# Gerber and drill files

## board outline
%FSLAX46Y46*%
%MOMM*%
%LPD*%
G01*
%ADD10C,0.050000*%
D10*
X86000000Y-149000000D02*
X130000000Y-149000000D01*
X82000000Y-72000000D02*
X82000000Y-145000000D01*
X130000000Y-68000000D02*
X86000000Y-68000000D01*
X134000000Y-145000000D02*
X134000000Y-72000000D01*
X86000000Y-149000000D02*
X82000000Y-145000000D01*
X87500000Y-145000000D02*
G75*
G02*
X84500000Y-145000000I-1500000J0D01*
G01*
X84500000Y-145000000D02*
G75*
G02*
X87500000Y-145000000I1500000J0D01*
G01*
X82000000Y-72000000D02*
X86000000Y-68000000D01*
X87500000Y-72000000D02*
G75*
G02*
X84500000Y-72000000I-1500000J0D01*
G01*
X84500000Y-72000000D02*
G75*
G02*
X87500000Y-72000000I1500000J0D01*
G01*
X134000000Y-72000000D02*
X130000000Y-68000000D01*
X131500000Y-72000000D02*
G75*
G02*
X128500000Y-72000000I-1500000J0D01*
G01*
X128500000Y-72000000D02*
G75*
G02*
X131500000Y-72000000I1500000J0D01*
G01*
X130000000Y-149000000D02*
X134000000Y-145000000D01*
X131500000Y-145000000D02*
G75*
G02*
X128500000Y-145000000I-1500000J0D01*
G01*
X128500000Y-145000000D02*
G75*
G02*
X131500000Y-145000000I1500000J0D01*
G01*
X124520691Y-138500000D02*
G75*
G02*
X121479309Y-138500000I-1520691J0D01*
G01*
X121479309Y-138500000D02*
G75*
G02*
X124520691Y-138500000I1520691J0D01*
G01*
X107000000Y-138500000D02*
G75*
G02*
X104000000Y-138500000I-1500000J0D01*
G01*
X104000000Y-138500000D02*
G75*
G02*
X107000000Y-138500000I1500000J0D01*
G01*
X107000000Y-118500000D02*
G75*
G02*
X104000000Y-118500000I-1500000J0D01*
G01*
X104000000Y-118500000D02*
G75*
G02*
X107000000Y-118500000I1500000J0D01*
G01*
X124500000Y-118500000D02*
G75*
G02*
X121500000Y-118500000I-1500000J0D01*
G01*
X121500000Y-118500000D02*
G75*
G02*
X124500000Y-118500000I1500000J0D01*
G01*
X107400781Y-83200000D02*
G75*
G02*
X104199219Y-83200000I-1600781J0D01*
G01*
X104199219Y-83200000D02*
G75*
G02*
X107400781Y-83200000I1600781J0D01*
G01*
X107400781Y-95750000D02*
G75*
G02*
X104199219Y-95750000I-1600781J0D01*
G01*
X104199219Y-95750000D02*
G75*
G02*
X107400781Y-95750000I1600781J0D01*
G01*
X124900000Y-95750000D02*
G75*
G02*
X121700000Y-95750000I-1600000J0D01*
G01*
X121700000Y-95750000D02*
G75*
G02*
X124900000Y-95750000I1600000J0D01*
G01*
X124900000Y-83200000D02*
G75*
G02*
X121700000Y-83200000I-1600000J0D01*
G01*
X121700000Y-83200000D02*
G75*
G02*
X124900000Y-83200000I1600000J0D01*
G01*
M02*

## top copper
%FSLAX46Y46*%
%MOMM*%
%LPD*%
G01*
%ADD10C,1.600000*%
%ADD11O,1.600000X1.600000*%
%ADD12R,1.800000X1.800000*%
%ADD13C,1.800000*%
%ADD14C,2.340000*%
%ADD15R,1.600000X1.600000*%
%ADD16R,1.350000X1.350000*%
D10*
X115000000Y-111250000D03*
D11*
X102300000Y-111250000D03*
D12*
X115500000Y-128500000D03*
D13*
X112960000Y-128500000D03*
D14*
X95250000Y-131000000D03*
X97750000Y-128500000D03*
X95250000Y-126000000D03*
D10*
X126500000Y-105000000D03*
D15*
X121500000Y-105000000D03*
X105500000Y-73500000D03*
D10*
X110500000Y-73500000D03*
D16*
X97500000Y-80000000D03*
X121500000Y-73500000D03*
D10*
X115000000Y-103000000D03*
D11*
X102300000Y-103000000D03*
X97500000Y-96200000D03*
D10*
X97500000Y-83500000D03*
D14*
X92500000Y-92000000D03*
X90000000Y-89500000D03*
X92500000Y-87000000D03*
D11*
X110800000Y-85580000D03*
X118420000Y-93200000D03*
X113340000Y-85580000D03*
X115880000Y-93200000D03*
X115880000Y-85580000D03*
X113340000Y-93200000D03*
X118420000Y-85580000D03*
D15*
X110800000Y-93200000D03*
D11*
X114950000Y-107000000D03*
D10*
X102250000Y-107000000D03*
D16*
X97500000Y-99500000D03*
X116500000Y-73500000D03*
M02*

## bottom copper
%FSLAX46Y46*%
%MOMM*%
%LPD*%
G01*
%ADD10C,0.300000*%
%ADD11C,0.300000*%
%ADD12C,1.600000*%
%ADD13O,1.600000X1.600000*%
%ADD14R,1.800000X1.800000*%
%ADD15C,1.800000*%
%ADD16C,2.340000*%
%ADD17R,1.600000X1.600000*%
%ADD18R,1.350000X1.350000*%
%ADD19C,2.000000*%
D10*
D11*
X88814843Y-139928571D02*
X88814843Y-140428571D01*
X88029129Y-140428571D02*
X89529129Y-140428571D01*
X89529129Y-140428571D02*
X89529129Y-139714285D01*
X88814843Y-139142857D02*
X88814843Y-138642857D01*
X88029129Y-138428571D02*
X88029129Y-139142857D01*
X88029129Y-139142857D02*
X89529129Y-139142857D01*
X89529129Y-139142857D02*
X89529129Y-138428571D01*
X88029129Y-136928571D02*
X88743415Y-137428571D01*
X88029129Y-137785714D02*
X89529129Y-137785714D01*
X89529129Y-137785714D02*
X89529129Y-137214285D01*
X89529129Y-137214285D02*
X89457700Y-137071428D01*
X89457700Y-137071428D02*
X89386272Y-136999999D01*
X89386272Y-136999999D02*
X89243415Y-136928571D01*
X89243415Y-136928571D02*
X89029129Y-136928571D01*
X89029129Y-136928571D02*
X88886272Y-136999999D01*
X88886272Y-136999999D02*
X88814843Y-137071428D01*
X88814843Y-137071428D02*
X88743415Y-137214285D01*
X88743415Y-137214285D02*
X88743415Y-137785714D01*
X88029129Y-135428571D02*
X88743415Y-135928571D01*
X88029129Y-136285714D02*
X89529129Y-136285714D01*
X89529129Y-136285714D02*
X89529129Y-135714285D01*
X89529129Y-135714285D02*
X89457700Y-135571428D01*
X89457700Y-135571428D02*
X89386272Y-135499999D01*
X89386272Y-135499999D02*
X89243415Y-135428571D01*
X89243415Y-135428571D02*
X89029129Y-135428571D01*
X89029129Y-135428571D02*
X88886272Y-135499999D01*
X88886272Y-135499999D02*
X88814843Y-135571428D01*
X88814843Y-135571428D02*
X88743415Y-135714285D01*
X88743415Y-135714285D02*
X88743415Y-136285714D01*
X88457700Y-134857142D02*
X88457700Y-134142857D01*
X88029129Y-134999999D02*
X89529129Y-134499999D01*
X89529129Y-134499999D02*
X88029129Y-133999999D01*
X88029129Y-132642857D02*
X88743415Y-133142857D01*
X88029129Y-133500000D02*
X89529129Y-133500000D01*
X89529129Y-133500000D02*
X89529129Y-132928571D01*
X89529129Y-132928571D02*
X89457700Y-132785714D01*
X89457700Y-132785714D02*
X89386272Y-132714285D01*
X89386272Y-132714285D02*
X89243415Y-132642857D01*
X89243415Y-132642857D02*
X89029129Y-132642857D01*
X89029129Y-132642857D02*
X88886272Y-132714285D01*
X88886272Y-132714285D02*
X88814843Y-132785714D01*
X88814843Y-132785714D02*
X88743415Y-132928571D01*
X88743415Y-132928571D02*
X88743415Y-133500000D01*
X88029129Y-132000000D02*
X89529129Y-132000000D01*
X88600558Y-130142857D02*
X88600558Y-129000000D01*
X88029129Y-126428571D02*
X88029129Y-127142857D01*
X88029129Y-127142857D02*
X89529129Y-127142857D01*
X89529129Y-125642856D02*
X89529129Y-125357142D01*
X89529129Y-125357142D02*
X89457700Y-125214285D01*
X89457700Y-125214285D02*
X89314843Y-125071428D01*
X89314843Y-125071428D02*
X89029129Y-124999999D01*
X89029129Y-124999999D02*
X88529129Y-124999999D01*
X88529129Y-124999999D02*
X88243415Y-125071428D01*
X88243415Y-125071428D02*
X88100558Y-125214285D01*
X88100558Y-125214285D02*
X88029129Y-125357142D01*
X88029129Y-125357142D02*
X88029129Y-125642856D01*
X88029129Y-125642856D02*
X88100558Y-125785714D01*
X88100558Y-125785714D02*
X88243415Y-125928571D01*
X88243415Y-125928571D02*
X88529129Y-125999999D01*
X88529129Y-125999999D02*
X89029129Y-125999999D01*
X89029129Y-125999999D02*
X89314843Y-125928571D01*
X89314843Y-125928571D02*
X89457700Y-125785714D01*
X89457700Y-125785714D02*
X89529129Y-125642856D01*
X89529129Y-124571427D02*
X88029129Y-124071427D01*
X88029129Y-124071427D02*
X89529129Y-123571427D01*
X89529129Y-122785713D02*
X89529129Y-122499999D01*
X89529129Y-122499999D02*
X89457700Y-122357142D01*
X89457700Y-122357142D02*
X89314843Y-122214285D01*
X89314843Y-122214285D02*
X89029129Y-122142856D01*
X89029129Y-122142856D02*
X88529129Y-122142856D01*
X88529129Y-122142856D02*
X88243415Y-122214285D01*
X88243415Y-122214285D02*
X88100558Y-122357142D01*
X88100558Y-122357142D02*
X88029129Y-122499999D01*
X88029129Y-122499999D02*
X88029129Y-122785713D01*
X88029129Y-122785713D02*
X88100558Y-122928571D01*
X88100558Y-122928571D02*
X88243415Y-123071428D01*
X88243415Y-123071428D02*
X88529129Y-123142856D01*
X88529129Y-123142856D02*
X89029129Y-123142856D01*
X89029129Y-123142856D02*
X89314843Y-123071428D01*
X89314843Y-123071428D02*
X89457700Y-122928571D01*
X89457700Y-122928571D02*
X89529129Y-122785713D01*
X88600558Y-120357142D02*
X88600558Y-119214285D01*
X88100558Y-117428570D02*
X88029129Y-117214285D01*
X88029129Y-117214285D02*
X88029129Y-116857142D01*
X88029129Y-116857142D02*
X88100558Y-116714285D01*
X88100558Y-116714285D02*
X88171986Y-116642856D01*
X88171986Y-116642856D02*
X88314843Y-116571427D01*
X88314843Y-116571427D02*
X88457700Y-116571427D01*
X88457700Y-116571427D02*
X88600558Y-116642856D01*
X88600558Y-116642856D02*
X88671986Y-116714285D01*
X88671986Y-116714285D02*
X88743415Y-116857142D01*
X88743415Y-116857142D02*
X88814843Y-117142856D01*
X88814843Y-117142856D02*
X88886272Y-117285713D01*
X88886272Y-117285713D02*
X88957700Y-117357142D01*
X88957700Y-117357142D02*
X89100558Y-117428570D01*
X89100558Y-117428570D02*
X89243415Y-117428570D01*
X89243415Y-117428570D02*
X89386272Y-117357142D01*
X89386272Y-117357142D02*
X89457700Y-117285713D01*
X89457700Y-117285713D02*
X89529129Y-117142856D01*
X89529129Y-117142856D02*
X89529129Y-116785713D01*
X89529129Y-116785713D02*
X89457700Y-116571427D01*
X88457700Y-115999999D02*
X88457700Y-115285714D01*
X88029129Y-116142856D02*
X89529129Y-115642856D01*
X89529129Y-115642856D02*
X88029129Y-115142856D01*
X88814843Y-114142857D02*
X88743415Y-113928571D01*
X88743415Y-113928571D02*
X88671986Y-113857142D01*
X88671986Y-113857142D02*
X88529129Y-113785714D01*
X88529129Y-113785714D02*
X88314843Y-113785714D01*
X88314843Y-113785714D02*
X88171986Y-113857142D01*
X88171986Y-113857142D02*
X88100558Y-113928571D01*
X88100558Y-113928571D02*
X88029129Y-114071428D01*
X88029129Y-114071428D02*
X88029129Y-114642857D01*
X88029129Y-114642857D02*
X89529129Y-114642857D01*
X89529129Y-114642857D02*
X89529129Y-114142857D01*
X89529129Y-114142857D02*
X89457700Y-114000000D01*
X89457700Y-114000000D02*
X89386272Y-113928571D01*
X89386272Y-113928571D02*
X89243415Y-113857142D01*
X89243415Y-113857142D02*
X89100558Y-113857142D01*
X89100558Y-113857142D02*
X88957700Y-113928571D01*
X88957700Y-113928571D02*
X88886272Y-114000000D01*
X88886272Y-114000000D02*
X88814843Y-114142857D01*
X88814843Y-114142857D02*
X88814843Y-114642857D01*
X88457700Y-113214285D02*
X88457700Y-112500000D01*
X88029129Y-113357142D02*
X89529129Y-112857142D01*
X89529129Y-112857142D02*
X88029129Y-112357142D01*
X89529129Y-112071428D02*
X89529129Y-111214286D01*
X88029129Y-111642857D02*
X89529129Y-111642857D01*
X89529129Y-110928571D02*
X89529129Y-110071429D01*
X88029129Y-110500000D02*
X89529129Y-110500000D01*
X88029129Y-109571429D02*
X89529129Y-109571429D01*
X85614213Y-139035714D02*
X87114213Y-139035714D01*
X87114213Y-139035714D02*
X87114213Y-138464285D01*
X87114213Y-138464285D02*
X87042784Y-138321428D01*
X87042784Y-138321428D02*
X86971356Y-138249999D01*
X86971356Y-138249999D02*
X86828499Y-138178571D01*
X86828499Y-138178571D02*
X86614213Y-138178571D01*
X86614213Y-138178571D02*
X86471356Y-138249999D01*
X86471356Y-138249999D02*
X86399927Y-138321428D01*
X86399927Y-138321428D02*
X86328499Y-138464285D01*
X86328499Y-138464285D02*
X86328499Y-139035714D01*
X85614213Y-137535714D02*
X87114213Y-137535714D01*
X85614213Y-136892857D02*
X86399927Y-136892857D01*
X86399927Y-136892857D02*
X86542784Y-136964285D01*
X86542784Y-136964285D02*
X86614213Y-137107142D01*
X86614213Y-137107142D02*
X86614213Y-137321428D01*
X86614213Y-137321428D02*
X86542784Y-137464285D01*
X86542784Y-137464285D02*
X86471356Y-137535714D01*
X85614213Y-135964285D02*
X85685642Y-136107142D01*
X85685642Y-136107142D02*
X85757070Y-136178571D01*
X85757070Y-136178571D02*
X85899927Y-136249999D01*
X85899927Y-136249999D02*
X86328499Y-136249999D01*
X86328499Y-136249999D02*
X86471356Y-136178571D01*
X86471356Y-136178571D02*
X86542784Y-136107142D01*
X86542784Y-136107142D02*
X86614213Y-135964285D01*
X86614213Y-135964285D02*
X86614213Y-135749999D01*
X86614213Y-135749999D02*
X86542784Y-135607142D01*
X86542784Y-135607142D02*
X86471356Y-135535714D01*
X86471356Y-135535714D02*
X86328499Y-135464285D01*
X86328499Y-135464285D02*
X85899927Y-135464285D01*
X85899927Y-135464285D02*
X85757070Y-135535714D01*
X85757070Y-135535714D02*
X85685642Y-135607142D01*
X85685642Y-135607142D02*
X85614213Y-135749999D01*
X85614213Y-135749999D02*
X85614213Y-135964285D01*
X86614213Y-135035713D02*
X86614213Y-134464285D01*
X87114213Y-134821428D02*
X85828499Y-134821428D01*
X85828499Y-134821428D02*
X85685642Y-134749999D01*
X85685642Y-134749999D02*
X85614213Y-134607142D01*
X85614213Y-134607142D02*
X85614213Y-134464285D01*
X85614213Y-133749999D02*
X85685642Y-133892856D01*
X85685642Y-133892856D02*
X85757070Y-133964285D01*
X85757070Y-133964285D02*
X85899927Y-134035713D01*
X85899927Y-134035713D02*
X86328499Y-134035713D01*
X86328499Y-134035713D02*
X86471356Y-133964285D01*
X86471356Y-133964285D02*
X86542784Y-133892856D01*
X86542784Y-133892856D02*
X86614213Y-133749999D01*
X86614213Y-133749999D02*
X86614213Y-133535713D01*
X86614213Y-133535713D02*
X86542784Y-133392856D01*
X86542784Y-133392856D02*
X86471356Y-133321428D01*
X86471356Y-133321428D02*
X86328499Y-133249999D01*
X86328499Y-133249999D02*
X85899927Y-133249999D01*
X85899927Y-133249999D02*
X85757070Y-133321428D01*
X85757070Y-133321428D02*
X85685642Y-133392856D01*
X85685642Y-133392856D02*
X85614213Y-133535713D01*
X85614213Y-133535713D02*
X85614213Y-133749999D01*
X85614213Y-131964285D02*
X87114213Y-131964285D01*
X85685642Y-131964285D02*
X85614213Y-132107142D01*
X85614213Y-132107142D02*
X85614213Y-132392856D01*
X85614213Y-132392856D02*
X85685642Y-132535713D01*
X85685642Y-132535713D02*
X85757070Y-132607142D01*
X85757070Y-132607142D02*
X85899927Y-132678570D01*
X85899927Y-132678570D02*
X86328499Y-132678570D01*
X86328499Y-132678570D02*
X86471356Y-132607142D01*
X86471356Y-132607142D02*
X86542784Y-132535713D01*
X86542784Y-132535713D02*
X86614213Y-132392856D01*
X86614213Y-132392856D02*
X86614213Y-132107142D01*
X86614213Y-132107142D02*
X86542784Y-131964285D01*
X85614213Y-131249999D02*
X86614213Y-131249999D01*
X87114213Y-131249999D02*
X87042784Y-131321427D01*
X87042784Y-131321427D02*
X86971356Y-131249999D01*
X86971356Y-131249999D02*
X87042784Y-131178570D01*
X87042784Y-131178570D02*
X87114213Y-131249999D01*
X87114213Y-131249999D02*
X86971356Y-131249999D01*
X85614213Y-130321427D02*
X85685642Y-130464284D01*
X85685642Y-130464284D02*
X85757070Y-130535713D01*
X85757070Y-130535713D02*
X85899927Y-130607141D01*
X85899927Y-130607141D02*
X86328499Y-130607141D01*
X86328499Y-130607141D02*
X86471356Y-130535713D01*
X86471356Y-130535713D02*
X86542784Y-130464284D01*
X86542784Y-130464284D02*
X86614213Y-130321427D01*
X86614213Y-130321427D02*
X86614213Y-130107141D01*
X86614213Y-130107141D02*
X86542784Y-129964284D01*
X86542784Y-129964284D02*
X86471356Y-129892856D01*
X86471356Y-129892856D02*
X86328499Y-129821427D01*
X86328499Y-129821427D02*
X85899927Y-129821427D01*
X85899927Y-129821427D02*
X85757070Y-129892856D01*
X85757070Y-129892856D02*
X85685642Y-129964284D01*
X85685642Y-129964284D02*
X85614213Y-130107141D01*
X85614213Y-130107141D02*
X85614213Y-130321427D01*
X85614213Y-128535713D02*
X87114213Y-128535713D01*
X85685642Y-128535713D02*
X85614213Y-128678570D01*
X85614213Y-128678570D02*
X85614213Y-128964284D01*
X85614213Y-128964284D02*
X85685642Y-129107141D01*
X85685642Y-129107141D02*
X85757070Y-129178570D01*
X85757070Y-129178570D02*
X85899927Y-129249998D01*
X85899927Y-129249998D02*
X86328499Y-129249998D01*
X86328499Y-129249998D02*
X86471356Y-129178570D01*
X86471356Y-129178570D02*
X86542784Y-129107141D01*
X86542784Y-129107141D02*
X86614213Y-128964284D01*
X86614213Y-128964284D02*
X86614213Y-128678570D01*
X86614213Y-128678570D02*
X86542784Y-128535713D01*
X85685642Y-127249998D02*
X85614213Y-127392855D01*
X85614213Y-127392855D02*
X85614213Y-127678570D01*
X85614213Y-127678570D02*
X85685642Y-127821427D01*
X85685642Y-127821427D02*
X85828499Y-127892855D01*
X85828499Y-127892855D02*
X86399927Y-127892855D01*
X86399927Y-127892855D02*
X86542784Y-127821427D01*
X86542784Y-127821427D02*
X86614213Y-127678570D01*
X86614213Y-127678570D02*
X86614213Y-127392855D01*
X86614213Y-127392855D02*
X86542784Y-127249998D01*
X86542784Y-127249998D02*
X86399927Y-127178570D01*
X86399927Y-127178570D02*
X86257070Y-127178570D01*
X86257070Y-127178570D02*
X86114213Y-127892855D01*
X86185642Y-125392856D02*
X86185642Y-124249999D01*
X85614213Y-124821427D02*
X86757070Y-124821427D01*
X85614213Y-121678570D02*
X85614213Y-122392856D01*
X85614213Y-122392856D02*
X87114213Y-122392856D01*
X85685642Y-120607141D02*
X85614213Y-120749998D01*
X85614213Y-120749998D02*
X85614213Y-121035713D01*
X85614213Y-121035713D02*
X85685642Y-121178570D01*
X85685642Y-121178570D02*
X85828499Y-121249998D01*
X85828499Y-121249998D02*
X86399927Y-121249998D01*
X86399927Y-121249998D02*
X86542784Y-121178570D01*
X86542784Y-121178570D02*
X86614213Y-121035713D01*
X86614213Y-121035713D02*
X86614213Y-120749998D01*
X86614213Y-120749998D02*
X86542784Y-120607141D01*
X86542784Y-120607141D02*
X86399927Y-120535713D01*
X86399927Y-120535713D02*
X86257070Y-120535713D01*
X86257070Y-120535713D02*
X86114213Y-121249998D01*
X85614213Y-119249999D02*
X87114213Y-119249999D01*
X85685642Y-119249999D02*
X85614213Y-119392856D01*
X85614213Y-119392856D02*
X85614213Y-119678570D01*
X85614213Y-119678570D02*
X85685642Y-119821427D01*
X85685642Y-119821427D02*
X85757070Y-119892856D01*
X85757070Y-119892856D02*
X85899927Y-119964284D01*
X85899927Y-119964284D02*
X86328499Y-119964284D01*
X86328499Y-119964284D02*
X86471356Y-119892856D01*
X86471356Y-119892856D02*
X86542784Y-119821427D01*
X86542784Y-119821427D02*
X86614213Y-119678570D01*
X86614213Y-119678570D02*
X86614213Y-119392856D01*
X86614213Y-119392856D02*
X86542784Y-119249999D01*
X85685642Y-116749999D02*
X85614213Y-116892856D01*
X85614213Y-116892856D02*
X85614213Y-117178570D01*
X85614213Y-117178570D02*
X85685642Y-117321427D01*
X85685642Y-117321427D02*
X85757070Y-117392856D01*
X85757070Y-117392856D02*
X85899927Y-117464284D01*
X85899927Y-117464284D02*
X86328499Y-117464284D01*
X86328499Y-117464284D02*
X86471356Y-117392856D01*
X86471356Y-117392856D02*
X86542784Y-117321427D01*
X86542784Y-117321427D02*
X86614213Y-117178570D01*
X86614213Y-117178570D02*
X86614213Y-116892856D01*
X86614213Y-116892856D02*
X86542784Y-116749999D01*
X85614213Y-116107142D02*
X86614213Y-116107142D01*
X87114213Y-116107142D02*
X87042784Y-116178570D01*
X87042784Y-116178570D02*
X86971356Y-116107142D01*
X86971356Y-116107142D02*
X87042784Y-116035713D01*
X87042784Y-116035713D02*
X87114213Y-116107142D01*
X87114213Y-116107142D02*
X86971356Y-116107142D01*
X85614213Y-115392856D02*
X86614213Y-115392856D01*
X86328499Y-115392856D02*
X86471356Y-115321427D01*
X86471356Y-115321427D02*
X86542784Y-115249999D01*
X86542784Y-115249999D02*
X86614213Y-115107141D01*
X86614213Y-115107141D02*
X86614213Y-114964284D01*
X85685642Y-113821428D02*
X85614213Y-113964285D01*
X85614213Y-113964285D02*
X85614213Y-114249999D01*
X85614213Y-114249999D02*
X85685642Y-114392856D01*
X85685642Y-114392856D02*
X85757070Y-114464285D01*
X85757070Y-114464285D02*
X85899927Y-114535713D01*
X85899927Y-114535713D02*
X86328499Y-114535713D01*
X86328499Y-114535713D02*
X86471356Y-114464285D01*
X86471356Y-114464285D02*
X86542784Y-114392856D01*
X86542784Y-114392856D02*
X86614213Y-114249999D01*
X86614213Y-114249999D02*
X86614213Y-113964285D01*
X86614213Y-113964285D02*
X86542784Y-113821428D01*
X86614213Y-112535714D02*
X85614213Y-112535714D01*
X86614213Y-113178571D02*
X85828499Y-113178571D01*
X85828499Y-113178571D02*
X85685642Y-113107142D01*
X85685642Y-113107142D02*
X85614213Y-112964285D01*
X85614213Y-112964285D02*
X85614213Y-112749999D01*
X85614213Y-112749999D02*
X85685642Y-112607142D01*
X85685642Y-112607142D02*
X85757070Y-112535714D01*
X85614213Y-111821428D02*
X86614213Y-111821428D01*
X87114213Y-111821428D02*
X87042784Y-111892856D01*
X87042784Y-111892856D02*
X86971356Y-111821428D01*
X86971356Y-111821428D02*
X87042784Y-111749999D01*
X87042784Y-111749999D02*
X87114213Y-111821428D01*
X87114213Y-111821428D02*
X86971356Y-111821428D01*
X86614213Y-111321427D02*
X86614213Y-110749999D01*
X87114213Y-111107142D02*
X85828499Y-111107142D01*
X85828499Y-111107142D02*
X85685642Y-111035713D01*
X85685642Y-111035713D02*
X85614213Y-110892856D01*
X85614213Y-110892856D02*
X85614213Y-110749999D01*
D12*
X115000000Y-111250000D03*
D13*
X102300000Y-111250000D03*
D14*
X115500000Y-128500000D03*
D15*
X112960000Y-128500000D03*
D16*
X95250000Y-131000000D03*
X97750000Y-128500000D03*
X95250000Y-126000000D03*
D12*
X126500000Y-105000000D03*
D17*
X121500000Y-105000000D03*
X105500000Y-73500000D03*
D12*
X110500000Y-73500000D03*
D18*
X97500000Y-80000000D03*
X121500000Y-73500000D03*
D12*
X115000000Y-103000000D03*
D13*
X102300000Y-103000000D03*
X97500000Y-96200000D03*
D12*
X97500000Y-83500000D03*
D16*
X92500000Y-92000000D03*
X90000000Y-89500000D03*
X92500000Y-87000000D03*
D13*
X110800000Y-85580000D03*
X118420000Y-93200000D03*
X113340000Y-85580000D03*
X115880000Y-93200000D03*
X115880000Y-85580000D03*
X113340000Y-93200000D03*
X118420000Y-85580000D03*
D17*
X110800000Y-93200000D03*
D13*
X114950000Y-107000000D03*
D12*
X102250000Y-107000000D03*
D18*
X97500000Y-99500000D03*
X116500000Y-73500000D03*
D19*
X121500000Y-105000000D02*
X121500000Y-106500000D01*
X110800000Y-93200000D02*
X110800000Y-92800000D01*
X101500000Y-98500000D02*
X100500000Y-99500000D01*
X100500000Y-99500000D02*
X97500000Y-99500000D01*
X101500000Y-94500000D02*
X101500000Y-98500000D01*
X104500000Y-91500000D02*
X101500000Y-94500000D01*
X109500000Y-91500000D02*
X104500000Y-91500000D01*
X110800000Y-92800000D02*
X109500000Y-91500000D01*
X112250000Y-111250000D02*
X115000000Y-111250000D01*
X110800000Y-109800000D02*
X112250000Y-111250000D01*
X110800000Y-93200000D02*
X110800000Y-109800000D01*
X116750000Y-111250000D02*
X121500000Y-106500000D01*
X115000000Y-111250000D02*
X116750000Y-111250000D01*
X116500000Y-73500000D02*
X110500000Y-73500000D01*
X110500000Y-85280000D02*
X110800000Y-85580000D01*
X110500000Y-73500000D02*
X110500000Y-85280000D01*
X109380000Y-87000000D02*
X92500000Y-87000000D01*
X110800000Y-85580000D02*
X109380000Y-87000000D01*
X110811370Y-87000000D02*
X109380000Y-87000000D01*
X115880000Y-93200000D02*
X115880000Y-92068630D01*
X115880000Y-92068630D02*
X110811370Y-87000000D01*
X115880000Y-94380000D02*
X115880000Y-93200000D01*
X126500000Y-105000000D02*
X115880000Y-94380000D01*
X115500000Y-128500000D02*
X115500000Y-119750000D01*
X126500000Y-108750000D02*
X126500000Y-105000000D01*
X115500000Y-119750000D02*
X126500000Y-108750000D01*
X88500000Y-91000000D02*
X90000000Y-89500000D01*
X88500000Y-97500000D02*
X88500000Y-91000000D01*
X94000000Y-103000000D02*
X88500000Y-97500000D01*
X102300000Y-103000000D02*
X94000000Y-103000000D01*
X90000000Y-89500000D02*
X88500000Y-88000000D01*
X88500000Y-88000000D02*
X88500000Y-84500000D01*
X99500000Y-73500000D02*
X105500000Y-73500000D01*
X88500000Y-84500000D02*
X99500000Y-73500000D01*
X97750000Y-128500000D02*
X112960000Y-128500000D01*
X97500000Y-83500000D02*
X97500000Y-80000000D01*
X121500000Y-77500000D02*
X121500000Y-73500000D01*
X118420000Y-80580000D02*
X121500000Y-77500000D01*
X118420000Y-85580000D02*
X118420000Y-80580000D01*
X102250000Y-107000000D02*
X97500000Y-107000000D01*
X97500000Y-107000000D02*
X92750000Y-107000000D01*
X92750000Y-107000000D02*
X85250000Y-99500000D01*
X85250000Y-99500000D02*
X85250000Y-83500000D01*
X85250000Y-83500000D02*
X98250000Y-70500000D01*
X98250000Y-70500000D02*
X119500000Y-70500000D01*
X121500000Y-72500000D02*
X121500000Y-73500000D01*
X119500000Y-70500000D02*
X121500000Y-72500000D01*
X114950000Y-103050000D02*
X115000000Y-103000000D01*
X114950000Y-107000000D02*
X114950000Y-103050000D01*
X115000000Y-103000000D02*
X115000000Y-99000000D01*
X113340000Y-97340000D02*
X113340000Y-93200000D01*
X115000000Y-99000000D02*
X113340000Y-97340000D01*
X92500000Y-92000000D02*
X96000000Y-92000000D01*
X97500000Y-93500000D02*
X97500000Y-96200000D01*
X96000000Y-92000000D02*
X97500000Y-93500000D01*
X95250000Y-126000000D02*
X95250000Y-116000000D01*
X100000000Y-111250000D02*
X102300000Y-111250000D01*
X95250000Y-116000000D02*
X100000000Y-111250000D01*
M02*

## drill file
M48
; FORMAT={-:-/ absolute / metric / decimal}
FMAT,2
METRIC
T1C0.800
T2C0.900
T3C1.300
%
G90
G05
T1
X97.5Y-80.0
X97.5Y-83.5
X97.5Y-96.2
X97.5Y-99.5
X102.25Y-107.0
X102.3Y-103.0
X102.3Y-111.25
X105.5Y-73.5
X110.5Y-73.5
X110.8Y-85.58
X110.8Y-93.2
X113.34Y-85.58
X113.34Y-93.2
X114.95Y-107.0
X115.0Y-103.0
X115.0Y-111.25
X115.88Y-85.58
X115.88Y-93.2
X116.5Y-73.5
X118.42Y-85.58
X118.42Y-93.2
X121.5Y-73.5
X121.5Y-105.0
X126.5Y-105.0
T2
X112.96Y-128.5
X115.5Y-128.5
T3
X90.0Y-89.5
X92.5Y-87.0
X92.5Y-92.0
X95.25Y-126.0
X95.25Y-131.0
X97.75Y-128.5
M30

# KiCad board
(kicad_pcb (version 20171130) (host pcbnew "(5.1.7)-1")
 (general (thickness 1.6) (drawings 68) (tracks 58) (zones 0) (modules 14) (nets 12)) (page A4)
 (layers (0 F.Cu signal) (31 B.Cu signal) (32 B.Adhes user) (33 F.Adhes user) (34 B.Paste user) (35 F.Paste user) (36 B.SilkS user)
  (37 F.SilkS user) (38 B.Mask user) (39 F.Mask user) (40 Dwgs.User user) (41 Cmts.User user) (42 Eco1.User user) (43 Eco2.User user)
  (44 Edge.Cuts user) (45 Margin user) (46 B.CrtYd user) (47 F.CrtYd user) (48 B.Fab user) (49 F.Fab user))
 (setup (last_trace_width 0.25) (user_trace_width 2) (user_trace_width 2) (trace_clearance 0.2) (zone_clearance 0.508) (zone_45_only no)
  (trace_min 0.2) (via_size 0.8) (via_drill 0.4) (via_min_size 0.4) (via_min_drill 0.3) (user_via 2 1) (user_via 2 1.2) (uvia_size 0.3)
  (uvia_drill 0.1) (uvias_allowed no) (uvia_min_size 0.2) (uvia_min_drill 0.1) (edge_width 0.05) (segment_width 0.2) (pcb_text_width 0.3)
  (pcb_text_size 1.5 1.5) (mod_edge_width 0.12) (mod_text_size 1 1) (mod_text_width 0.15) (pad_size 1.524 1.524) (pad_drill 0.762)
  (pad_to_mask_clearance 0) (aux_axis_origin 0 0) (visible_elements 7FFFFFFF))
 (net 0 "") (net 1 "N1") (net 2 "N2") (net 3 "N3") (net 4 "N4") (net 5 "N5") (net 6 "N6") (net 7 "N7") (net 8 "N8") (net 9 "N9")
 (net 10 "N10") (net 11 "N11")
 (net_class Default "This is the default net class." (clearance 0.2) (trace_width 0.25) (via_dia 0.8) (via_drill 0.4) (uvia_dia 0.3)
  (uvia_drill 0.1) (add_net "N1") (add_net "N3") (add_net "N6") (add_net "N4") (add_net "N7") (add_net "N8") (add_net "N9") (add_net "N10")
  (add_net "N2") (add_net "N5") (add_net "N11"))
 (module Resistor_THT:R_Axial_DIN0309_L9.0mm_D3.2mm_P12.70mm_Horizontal (layer F.Cu) (at 115 111.25 180)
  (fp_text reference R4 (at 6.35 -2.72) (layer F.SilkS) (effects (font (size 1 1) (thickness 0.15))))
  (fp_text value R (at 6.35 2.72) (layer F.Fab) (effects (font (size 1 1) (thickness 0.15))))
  (pad 1 thru_hole circle (at 0 0 180) (size 1.6 1.6) (drill 0.8) (layers *.Cu *.Mask) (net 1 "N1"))
  (pad 2 thru_hole oval (at 12.7 0 180) (size 1.6 1.6) (drill 0.8) (layers *.Cu *.Mask) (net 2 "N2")))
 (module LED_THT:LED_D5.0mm (layer F.Cu) (at 115.5 128.5 180)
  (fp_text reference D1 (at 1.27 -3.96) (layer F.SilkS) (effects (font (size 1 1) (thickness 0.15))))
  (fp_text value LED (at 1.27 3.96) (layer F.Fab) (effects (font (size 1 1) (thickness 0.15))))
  (pad 1 thru_hole rect (at 0 0 180) (size 1.8 1.8) (drill 0.9) (layers *.Cu *.Mask) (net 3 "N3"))
  (pad 2 thru_hole circle (at 2.54 0 180) (size 1.8 1.8) (drill 0.9) (layers *.Cu *.Mask) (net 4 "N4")))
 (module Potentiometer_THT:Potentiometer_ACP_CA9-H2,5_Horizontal (layer F.Cu) (at 95.25 126)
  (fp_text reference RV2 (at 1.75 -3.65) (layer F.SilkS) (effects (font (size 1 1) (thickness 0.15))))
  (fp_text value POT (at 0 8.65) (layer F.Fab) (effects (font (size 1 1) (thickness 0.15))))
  (pad 3 thru_hole circle (at 0 5) (size 2.34 2.34) (drill 1.3) (layers *.Cu *.Mask) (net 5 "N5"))
  (pad 2 thru_hole circle (at 2.5 2.5) (size 2.34 2.34) (drill 1.3) (layers *.Cu *.Mask) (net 4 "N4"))
  (pad 1 thru_hole circle (at 0 0) (size 2.34 2.34) (drill 1.3) (layers *.Cu *.Mask) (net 2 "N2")))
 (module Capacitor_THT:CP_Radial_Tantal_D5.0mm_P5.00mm (layer F.Cu) (at 121.5 105)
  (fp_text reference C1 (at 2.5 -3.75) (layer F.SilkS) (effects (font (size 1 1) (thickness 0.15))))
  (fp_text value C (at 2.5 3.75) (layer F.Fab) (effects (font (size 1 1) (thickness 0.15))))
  (pad 2 thru_hole circle (at 5 0) (size 1.6 1.6) (drill 0.8) (layers *.Cu *.Mask) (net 3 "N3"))
  (pad 1 thru_hole rect (at 0 0) (size 1.6 1.6) (drill 0.8) (layers *.Cu *.Mask) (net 1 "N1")))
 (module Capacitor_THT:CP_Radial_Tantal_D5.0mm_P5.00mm (layer F.Cu) (at 105.5 73.5)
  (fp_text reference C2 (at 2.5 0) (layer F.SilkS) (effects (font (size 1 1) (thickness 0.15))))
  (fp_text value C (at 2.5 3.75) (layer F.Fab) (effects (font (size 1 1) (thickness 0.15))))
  (pad 1 thru_hole rect (at 0 0) (size 1.6 1.6) (drill 0.8) (layers *.Cu *.Mask) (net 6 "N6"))
  (pad 2 thru_hole circle (at 5 0) (size 1.6 1.6) (drill 0.8) (layers *.Cu *.Mask) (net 3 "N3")))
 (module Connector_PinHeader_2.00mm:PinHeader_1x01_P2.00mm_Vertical (layer F.Cu) (at 97.5 80)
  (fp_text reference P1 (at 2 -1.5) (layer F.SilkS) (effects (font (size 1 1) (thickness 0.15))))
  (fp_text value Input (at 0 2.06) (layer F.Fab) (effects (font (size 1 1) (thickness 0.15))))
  (pad 1 thru_hole rect (at 0 0) (size 1.35 1.35) (drill 0.8) (layers *.Cu *.Mask) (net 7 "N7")))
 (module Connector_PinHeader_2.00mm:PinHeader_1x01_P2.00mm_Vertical (layer F.Cu) (at 121.5 73.5)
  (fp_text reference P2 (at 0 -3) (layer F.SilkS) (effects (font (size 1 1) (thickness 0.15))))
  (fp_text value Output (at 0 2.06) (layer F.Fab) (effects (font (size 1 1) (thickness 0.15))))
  (pad 1 thru_hole rect (at 0 0) (size 1.35 1.35) (drill 0.8) (layers *.Cu *.Mask) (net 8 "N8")))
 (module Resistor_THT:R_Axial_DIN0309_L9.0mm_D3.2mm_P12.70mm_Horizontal (layer F.Cu) (at 115 103 180)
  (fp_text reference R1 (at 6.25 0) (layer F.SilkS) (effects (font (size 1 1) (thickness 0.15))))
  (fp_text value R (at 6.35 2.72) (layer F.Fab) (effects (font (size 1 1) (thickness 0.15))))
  (pad 1 thru_hole circle (at 0 0 180) (size 1.6 1.6) (drill 0.8) (layers *.Cu *.Mask) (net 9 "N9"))
  (pad 2 thru_hole oval (at 12.7 0 180) (size 1.6 1.6) (drill 0.8) (layers *.Cu *.Mask) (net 6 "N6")))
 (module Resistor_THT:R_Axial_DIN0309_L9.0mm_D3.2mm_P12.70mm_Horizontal (layer F.Cu) (at 97.5 83.5 270)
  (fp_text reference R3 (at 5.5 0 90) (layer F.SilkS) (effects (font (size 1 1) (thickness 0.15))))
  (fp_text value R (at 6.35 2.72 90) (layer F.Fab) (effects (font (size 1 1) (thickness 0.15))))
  (pad 2 thru_hole oval (at 12.7 0 270) (size 1.6 1.6) (drill 0.8) (layers *.Cu *.Mask) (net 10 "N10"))
  (pad 1 thru_hole circle (at 0 0 270) (size 1.6 1.6) (drill 0.8) (layers *.Cu *.Mask) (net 7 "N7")))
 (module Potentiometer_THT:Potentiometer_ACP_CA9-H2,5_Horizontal (layer F.Cu) (at 92.5 92 180)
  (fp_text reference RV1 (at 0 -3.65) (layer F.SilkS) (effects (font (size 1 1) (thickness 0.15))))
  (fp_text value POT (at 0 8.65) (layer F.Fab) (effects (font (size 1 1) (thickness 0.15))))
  (pad 1 thru_hole circle (at 0 0 180) (size 2.34 2.34) (drill 1.3) (layers *.Cu *.Mask) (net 10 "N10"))
  (pad 2 thru_hole circle (at 2.5 2.5 180) (size 2.34 2.34) (drill 1.3) (layers *.Cu *.Mask) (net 6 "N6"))
  (pad 3 thru_hole circle (at 0 5 180) (size 2.34 2.34) (drill 1.3) (layers *.Cu *.Mask) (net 3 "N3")))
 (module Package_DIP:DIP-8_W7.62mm (layer F.Cu) (at 110.8 93.2 90)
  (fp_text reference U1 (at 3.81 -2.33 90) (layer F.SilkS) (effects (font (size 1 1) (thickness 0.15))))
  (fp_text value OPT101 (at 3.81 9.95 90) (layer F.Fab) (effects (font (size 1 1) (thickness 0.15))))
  (pad 8 thru_hole oval (at 7.62 0 90) (size 1.6 1.6) (drill 0.8) (layers *.Cu *.Mask) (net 3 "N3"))
  (pad 4 thru_hole oval (at 0 7.62 90) (size 1.6 1.6) (drill 0.8) (layers *.Cu *.Mask) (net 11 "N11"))
  (pad 7 thru_hole oval (at 7.62 2.54 90) (size 1.6 1.6) (drill 0.8) (layers *.Cu *.Mask))
  (pad 3 thru_hole oval (at 0 5.08 90) (size 1.6 1.6) (drill 0.8) (layers *.Cu *.Mask) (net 3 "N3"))
  (pad 6 thru_hole oval (at 7.62 5.08 90) (size 1.6 1.6) (drill 0.8) (layers *.Cu *.Mask))
  (pad 2 thru_hole oval (at 0 2.54 90) (size 1.6 1.6) (drill 0.8) (layers *.Cu *.Mask) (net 9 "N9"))
  (pad 5 thru_hole oval (at 7.62 7.62 90) (size 1.6 1.6) (drill 0.8) (layers *.Cu *.Mask) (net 8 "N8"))
  (pad 1 thru_hole rect (at 0 0 90) (size 1.6 1.6) (drill 0.8) (layers *.Cu *.Mask) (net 1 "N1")))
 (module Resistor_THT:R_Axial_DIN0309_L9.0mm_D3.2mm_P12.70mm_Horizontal (layer F.Cu) (at 102.25 107)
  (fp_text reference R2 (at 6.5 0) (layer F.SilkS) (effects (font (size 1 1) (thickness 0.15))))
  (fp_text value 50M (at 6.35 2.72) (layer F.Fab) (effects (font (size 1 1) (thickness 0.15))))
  (pad 2 thru_hole oval (at 12.7 0) (size 1.6 1.6) (drill 0.8) (layers *.Cu *.Mask) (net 9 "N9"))
  (pad 1 thru_hole circle (at 0 0) (size 1.6 1.6) (drill 0.8) (layers *.Cu *.Mask) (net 8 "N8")))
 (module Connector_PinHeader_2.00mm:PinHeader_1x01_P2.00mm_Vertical (layer F.Cu) (at 97.5 99.5 180)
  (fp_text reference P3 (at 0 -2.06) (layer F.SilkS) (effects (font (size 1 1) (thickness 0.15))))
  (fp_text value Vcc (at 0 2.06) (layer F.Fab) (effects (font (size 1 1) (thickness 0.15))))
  (pad 1 thru_hole rect (at 0 0 180) (size 1.35 1.35) (drill 0.8) (layers *.Cu *.Mask) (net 1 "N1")))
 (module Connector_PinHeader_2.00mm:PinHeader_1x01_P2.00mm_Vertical (layer F.Cu) (at 116.5 73.5 180)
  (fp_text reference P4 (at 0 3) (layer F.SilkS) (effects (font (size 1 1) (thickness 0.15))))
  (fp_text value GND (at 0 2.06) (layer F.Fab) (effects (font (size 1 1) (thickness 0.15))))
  (pad 1 thru_hole rect (at 0 0 180) (size 1.35 1.35) (drill 0.8) (layers *.Cu *.Mask) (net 3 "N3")))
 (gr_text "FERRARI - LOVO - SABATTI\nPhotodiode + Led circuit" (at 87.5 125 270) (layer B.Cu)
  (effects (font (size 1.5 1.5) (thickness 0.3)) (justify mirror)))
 (gr_line (start 86 149) (end 130 149) (layer Edge.Cuts) (width 0.05))
 (gr_line (start 82 72) (end 82 145) (layer Edge.Cuts) (width 0.05))
 (gr_line (start 130 68) (end 86 68) (layer Edge.Cuts) (width 0.05))
 (gr_line (start 134 145) (end 134 72) (layer Edge.Cuts) (width 0.05))
 (gr_line (start 86 149) (end 82 145) (layer Edge.Cuts) (width 0.05))
 (gr_circle (center 86 145) (end 87.5 145) (layer Edge.Cuts) (width 0.05))
 (gr_line (start 82 72) (end 86 68) (layer Edge.Cuts) (width 0.05))
 (gr_circle (center 86 72) (end 87.5 72) (layer Edge.Cuts) (width 0.05))
 (gr_line (start 134 72) (end 130 68) (layer Edge.Cuts) (width 0.05))
 (gr_circle (center 130 72) (end 131.5 72) (layer Edge.Cuts) (width 0.05))
 (gr_line (start 130 149) (end 134 145) (layer Edge.Cuts) (width 0.05))
 (gr_circle (center 130 145) (end 128.5 145) (layer Edge.Cuts) (width 0.05))
 (gr_circle (center 123 138.5) (end 124.5 138.25) (layer Edge.Cuts) (width 0.05))
 (gr_circle (center 105.5 138.5) (end 104 138.5) (layer Edge.Cuts) (width 0.05))
 (gr_circle (center 105.5 118.5) (end 107 118.5) (layer Edge.Cuts) (width 0.05))
 (gr_circle (center 123 118.5) (end 121.5 118.5) (layer Edge.Cuts) (width 0.05))
 (gr_circle (center 105.8 83.2) (end 104.2 83.15) (layer Edge.Cuts) (width 0.05))
 (gr_circle (center 105.8 95.75) (end 104.2 95.8) (layer Edge.Cuts) (width 0.05))
 (gr_circle (center 123.3 95.75) (end 121.7 95.75) (layer Edge.Cuts) (width 0.05))
 (gr_circle (center 123.3 83.2) (end 121.7 83.2) (layer Edge.Cuts) (width 0.05))
 (segment (start 121.5 105) (end 121.5 106.5) (width 2) (layer B.Cu) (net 1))
 (segment (start 110.8 93.2) (end 110.8 92.8) (width 2) (layer B.Cu) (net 1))
 (segment (start 101.5 98.5) (end 100.5 99.5) (width 2) (layer B.Cu) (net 1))
 (segment (start 100.5 99.5) (end 97.5 99.5) (width 2) (layer B.Cu) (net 1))
 (segment (start 101.5 94.5) (end 101.5 98.5) (width 2) (layer B.Cu) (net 1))
 (segment (start 104.5 91.5) (end 101.5 94.5) (width 2) (layer B.Cu) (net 1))
 (segment (start 109.5 91.5) (end 104.5 91.5) (width 2) (layer B.Cu) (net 1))
 (segment (start 110.8 92.8) (end 109.5 91.5) (width 2) (layer B.Cu) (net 1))
 (segment (start 112.25 111.25) (end 115 111.25) (width 2) (layer B.Cu) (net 1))
 (segment (start 110.8 109.8) (end 112.25 111.25) (width 2) (layer B.Cu) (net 1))
 (segment (start 110.8 93.2) (end 110.8 109.8) (width 2) (layer B.Cu) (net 1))
 (segment (start 116.75 111.25) (end 121.5 106.5) (width 2) (layer B.Cu) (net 1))
 (segment (start 115 111.25) (end 116.75 111.25) (width 2) (layer B.Cu) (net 1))
 (segment (start 116.5 73.5) (end 110.5 73.5) (width 2) (layer B.Cu) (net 3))
 (segment (start 110.5 85.28) (end 110.8 85.58) (width 2) (layer B.Cu) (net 3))
 (segment (start 110.5 73.5) (end 110.5 85.28) (width 2) (layer B.Cu) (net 3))
 (segment (start 109.38 87) (end 92.5 87) (width 2) (layer B.Cu) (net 3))
 (segment (start 110.8 85.58) (end 109.38 87) (width 2) (layer B.Cu) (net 3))
 (segment (start 110.81137 87) (end 109.38 87) (width 2) (layer B.Cu) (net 3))
 (segment (start 115.88 93.2) (end 115.88 92.06863) (width 2) (layer B.Cu) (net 3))
 (segment (start 115.88 92.06863) (end 110.81137 87) (width 2) (layer B.Cu) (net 3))
 (segment (start 115.88 94.38) (end 115.88 93.2) (width 2) (layer B.Cu) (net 3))
 (segment (start 126.5 105) (end 115.88 94.38) (width 2) (layer B.Cu) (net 3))
 (segment (start 115.5 128.5) (end 115.5 119.75) (width 2) (layer B.Cu) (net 3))
 (segment (start 126.5 108.75) (end 126.5 105) (width 2) (layer B.Cu) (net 3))
 (segment (start 115.5 119.75) (end 126.5 108.75) (width 2) (layer B.Cu) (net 3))
 (segment (start 88.5 91) (end 90 89.5) (width 2) (layer B.Cu) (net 6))
 (segment (start 88.5 97.5) (end 88.5 91) (width 2) (layer B.Cu) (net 6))
 (segment (start 94 103) (end 88.5 97.5) (width 2) (layer B.Cu) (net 6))
 (segment (start 102.3 103) (end 94 103) (width 2) (layer B.Cu) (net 6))
 (segment (start 90 89.5) (end 88.5 88) (width 2) (layer B.Cu) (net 6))
 (segment (start 88.5 88) (end 88.5 84.5) (width 2) (layer B.Cu) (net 6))
 (segment (start 99.5 73.5) (end 105.5 73.5) (width 2) (layer B.Cu) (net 6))
 (segment (start 88.5 84.5) (end 99.5 73.5) (width 2) (layer B.Cu) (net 6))
 (segment (start 97.75 128.5) (end 112.96 128.5) (width 2) (layer B.Cu) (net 4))
 (segment (start 97.5 83.5) (end 97.5 80) (width 2) (layer B.Cu) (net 7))
 (segment (start 121.5 77.5) (end 121.5 73.5) (width 2) (layer B.Cu) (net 8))
 (segment (start 118.42 80.58) (end 121.5 77.5) (width 2) (layer B.Cu) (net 8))
 (segment (start 118.42 85.58) (end 118.42 80.58) (width 2) (layer B.Cu) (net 8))
 (segment (start 102.25 107) (end 97.5 107) (width 2) (layer B.Cu) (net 8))
 (segment (start 97.5 107) (end 92.75 107) (width 2) (layer B.Cu) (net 8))
 (segment (start 92.75 107) (end 85.25 99.5) (width 2) (layer B.Cu) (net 8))
 (segment (start 85.25 99.5) (end 85.25 83.5) (width 2) (layer B.Cu) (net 8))
 (segment (start 85.25 83.5) (end 98.25 70.5) (width 2) (layer B.Cu) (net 8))
 (segment (start 98.25 70.5) (end 119.5 70.5) (width 2) (layer B.Cu) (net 8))
 (segment (start 121.5 72.5) (end 121.5 73.5) (width 2) (layer B.Cu) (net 8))
 (segment (start 119.5 70.5) (end 121.5 72.5) (width 2) (layer B.Cu) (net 8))
 (segment (start 114.95 103.05) (end 115 103) (width 2) (layer B.Cu) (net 9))
 (segment (start 114.95 107) (end 114.95 103.05) (width 2) (layer B.Cu) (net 9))
 (segment (start 115 103) (end 115 99) (width 2) (layer B.Cu) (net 9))
 (segment (start 113.34 97.34) (end 113.34 93.2) (width 2) (layer B.Cu) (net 9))
 (segment (start 115 99) (end 113.34 97.34) (width 2) (layer B.Cu) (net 9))
 (segment (start 92.5 92) (end 96 92) (width 2) (layer B.Cu) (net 10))
 (segment (start 97.5 93.5) (end 97.5 96.2) (width 2) (layer B.Cu) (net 10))
 (segment (start 96 92) (end 97.5 93.5) (width 2) (layer B.Cu) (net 10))
 (segment (start 95.25 126) (end 95.25 116) (width 2) (layer B.Cu) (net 2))
 (segment (start 100 111.25) (end 102.3 111.25) (width 2) (layer B.Cu) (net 2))
 (segment (start 95.25 116) (end 100 111.25) (width 2) (layer B.Cu) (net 2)))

